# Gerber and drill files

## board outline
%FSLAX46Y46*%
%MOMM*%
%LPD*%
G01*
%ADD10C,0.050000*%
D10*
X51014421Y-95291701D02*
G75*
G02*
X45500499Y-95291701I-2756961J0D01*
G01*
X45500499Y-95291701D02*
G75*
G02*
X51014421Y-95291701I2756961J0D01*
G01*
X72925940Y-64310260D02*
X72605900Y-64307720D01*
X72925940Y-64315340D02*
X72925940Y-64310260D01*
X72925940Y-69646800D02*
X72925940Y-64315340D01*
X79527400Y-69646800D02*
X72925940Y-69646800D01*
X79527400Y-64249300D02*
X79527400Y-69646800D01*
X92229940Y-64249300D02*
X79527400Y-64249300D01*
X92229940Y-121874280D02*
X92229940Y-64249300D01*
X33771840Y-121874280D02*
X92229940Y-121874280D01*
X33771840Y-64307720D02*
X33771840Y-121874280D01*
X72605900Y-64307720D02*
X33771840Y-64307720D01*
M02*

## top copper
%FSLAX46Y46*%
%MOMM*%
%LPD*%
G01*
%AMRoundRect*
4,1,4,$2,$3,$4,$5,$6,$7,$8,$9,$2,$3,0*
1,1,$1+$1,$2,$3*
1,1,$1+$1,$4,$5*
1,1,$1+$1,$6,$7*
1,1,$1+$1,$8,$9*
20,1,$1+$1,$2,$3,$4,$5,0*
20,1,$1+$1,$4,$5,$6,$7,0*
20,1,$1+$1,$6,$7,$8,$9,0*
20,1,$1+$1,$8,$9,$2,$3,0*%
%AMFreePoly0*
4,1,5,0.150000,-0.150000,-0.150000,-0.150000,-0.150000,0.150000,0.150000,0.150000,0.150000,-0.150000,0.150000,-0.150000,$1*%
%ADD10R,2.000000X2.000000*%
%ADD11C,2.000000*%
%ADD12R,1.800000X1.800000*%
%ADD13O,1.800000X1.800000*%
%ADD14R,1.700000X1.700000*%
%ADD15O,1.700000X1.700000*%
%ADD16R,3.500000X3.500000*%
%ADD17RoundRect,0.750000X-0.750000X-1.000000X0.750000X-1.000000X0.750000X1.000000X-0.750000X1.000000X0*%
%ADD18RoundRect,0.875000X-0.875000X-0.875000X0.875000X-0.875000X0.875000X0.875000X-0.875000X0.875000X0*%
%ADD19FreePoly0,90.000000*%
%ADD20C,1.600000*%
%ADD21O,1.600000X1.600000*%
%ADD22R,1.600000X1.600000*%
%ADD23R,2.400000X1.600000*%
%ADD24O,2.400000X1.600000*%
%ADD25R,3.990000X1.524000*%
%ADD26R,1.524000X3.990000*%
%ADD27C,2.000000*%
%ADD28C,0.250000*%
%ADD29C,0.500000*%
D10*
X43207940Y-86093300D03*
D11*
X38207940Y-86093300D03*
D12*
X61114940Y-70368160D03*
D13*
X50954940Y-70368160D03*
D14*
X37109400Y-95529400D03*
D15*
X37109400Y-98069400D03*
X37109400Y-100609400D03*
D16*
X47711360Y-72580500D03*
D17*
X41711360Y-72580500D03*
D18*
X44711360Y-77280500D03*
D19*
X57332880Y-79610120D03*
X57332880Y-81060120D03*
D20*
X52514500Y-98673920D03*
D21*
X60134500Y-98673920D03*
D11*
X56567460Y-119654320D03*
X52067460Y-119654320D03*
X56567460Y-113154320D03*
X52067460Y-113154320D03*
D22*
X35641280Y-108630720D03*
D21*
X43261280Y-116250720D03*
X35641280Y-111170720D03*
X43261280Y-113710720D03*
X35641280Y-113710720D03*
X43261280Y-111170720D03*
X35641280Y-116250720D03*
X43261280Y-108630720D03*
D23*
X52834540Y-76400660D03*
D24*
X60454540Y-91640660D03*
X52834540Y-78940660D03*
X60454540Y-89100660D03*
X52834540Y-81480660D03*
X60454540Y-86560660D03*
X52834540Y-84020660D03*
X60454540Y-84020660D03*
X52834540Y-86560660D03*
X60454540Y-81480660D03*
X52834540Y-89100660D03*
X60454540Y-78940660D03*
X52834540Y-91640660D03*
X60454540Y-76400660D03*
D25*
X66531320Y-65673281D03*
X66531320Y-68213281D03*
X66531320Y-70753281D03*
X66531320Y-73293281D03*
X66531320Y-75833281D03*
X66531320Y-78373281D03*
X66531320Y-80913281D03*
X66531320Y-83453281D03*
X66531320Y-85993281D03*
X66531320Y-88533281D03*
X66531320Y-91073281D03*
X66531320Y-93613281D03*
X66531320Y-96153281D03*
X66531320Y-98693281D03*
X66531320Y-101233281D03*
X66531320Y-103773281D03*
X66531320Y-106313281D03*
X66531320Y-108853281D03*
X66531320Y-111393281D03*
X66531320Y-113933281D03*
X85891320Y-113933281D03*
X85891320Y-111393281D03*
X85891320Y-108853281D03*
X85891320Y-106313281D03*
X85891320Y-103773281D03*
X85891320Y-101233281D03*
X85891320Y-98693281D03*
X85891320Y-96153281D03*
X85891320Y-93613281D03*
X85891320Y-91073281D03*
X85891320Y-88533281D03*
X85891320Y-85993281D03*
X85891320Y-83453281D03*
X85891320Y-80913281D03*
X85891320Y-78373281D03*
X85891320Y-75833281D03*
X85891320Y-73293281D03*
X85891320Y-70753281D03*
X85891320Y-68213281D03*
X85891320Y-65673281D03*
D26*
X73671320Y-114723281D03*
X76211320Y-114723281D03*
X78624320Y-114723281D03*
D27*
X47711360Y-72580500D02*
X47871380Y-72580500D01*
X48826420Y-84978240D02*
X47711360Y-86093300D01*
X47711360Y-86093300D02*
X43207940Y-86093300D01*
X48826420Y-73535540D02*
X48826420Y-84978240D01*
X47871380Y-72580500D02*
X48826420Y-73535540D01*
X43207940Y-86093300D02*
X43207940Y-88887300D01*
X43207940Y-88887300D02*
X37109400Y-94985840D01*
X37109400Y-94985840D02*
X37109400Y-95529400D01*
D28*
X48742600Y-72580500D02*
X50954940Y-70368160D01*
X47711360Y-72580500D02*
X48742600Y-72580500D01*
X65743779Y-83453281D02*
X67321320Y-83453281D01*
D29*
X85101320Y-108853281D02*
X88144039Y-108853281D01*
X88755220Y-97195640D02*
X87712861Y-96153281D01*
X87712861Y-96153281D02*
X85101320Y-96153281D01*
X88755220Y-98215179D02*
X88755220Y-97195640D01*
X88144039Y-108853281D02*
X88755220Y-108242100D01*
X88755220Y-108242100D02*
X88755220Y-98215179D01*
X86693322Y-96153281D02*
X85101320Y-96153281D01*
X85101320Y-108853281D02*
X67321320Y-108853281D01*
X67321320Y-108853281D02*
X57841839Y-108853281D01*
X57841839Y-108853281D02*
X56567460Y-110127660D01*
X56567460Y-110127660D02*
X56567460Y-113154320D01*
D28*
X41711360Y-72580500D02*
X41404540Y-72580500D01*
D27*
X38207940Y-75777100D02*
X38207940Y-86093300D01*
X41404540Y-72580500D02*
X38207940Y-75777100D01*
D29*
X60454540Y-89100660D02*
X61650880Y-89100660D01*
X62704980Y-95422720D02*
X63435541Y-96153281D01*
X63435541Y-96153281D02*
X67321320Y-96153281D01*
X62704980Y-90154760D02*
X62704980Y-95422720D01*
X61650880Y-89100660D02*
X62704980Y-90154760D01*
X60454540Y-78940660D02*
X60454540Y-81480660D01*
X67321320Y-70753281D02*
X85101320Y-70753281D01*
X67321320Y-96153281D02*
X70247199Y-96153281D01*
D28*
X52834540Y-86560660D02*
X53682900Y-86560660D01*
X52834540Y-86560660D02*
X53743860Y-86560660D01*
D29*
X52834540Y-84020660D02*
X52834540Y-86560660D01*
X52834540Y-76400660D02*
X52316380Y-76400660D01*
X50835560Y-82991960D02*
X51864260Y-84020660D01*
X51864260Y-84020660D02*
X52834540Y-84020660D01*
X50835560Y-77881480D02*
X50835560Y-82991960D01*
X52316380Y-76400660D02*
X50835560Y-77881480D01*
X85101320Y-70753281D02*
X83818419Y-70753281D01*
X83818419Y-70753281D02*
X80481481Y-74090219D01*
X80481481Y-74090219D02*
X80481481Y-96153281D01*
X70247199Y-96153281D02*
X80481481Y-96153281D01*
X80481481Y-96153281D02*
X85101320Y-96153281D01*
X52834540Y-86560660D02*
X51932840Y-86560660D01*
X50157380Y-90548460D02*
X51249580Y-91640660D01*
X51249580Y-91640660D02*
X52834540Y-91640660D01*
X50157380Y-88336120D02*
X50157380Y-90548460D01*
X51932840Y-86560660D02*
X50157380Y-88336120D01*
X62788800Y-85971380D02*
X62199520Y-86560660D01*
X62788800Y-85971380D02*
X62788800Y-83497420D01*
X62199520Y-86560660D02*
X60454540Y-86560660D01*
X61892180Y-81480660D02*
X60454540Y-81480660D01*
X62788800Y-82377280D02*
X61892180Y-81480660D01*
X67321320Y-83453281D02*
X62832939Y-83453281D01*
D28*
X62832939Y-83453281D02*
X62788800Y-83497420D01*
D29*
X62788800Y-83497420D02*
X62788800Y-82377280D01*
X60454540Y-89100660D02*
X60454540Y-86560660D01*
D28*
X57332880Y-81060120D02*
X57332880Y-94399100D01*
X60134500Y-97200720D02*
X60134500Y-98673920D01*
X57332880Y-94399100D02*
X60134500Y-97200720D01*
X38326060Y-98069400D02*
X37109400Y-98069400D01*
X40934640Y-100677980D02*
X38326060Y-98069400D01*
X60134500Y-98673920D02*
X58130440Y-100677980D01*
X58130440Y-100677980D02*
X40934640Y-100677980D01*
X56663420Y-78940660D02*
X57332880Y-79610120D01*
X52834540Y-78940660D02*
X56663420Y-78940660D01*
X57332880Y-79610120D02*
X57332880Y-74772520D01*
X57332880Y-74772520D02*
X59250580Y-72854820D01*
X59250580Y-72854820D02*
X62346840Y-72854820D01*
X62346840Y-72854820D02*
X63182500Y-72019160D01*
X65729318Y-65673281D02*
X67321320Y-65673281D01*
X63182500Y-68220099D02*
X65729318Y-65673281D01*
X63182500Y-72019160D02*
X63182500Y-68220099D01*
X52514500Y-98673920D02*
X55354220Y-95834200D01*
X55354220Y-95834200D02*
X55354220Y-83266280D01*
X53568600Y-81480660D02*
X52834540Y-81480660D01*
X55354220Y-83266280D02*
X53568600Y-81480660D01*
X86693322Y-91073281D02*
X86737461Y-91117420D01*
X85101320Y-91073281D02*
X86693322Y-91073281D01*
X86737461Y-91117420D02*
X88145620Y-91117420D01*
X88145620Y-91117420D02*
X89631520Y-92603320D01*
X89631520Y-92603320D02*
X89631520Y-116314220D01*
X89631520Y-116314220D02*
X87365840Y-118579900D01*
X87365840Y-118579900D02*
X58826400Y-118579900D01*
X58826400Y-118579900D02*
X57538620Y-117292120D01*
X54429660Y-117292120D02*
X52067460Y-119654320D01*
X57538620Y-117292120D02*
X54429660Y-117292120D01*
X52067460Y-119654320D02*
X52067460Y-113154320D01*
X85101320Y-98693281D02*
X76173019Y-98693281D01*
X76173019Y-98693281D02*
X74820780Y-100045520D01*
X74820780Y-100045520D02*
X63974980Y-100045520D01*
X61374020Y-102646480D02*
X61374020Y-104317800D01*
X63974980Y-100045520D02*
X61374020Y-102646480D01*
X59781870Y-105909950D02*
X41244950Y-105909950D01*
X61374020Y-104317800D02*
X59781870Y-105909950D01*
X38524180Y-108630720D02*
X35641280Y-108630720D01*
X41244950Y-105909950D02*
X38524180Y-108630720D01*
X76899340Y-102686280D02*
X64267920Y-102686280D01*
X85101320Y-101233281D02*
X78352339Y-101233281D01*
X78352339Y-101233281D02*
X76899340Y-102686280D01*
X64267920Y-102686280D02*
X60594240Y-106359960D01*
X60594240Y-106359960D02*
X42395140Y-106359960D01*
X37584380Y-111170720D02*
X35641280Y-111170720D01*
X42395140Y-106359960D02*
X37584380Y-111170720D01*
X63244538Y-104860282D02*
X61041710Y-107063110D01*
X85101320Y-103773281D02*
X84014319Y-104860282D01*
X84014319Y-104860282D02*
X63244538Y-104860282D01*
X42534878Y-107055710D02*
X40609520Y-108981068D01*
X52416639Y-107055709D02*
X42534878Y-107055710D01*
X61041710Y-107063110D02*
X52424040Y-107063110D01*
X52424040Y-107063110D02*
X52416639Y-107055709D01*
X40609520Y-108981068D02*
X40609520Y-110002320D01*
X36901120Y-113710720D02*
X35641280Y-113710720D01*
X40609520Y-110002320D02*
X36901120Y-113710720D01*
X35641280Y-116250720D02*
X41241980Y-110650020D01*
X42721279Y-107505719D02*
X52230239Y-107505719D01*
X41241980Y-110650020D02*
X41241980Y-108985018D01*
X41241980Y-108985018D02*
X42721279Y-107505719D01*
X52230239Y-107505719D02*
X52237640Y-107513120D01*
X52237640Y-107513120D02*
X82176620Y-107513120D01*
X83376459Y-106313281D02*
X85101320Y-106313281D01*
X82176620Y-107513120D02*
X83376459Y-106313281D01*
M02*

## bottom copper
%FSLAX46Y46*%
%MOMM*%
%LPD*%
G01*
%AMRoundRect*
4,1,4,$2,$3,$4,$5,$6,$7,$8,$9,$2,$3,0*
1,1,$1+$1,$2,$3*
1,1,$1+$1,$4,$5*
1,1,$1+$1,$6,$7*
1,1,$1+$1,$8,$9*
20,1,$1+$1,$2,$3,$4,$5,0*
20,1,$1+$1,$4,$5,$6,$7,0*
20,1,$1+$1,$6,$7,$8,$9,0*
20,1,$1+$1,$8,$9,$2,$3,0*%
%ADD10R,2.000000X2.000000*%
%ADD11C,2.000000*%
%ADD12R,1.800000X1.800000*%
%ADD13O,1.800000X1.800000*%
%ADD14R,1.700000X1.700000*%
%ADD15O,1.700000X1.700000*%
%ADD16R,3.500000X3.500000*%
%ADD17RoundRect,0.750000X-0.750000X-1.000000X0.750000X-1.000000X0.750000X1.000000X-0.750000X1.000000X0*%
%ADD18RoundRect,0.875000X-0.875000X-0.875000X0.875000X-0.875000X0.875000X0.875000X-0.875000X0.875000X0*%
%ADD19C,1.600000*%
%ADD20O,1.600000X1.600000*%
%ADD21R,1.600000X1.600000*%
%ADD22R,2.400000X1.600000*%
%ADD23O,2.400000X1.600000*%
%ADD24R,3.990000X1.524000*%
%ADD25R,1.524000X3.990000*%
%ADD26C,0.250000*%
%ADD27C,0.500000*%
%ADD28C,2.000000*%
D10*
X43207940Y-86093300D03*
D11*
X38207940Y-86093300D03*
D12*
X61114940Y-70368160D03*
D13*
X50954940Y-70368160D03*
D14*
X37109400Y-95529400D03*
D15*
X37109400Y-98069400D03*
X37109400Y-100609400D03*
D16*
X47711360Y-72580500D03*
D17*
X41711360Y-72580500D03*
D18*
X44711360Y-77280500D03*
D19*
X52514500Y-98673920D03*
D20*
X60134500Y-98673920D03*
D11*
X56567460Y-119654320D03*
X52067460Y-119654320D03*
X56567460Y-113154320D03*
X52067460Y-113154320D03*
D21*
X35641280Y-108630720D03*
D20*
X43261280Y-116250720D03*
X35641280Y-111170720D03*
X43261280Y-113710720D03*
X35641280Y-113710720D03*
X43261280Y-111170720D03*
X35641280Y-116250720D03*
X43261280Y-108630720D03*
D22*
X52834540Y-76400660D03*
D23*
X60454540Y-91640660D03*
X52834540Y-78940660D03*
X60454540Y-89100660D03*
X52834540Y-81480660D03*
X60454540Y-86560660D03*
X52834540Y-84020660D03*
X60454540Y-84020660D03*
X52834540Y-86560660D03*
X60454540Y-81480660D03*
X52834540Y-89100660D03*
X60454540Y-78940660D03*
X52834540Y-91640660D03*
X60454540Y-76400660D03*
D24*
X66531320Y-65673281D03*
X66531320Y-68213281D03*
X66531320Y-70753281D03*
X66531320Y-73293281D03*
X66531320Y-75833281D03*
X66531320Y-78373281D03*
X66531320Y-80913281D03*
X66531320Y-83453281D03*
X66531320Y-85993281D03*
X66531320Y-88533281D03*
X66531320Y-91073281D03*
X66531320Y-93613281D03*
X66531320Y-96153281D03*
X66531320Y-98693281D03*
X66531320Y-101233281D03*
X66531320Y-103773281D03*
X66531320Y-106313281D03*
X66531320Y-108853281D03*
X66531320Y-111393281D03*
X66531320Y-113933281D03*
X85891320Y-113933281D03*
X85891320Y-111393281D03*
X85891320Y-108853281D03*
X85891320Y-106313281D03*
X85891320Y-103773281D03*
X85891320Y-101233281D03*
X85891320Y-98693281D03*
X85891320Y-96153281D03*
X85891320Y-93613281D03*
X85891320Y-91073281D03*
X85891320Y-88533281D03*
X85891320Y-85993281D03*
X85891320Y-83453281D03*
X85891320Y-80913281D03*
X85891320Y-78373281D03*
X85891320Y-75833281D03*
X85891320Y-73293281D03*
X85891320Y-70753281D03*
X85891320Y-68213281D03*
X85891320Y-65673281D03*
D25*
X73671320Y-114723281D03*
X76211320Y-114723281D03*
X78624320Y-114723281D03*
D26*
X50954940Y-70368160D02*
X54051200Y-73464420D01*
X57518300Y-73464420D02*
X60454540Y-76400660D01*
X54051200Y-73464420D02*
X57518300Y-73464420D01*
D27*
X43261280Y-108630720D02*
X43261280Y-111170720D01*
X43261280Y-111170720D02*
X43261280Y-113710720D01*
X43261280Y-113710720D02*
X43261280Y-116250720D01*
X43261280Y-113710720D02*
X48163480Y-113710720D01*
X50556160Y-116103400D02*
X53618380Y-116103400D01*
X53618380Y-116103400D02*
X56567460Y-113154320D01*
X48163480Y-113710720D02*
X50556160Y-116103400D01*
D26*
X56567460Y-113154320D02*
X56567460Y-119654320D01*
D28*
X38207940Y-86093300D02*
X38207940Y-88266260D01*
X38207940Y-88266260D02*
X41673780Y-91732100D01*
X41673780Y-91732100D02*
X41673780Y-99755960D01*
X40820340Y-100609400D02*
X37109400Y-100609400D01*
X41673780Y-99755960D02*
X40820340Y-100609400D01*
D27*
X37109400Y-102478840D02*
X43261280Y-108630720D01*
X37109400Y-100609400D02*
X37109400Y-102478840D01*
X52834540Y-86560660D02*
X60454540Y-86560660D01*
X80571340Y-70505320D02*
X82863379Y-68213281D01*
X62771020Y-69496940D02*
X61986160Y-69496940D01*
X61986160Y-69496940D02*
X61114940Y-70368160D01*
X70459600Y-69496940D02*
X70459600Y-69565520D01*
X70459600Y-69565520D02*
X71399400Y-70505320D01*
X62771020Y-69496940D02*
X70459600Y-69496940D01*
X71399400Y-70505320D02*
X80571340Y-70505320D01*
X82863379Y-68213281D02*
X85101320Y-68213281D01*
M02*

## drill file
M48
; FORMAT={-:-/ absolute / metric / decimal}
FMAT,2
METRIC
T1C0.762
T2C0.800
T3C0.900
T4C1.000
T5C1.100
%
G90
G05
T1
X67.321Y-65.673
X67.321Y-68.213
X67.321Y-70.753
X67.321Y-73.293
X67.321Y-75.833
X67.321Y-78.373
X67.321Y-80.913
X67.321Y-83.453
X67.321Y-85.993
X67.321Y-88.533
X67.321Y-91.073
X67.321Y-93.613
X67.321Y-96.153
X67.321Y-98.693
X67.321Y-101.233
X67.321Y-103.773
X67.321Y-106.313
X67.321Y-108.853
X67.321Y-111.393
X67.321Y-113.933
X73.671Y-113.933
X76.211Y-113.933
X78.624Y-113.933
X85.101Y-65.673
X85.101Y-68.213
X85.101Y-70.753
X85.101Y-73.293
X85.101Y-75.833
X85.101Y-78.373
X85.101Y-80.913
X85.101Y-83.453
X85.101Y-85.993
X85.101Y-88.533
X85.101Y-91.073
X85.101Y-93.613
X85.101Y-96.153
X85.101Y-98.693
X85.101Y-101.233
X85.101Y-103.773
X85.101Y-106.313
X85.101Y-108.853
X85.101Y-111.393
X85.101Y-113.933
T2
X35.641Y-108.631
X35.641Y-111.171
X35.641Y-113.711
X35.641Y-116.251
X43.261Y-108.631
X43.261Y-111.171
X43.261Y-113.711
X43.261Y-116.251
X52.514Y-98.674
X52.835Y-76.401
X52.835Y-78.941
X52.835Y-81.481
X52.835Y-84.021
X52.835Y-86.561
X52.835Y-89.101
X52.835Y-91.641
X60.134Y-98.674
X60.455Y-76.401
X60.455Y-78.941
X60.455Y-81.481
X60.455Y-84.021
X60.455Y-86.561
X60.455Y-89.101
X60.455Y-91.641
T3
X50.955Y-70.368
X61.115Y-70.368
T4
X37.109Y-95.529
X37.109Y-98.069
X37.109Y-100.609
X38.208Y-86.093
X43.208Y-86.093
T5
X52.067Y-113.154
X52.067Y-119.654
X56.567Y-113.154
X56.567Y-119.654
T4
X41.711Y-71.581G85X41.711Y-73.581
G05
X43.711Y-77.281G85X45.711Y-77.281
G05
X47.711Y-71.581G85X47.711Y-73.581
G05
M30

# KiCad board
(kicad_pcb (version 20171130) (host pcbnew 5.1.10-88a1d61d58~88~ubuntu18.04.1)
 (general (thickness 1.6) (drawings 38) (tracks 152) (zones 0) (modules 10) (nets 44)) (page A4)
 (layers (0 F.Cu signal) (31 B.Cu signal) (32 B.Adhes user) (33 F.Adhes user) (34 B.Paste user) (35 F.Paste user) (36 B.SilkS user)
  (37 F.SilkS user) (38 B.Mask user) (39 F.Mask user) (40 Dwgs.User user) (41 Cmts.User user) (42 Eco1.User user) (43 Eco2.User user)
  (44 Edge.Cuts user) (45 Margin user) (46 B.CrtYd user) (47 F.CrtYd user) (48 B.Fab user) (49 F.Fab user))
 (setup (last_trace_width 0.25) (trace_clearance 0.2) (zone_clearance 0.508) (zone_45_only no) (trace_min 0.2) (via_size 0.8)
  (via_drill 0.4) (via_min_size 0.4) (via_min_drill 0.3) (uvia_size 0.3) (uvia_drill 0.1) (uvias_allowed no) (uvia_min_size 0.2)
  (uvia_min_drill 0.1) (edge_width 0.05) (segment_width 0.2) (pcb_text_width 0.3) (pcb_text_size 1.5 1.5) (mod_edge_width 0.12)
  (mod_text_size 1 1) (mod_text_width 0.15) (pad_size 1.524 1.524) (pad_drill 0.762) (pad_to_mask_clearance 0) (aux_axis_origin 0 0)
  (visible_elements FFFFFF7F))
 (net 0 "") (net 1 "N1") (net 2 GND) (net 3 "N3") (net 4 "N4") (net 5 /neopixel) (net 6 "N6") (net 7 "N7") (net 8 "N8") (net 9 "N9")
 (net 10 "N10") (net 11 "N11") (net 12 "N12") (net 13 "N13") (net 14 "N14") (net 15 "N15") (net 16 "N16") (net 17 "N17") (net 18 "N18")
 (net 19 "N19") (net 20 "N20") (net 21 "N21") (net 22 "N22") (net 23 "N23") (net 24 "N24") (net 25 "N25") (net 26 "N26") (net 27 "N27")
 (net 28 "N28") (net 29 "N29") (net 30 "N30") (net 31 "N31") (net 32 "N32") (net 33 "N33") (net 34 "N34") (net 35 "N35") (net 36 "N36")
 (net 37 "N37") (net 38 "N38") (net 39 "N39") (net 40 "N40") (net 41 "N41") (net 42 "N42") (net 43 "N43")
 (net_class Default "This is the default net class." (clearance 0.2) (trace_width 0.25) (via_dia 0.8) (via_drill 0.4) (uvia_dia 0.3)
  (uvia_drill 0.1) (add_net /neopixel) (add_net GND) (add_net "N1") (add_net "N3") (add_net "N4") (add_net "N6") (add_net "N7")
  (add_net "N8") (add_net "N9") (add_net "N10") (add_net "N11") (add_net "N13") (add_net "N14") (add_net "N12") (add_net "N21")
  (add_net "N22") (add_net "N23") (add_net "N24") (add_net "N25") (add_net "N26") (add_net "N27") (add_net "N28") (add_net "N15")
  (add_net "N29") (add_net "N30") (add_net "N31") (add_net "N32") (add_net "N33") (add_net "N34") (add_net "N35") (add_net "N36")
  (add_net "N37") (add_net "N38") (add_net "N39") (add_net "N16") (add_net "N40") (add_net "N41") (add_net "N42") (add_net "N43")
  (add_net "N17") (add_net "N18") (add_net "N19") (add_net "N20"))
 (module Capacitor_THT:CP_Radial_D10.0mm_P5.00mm (layer F.Cu) (at 43.20794 86.0933 180)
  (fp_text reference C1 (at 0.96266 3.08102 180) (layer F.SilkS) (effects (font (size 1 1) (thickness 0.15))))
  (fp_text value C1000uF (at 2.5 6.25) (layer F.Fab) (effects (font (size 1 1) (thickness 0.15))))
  (pad 1 thru_hole rect (at 0 0 180) (size 2 2) (drill 1) (layers *.Cu *.Mask) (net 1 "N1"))
  (pad 2 thru_hole circle (at 5 0 180) (size 2 2) (drill 1) (layers *.Cu *.Mask) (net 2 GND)))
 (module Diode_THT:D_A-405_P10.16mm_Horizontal (layer F.Cu) (at 61.11494 70.36816 180)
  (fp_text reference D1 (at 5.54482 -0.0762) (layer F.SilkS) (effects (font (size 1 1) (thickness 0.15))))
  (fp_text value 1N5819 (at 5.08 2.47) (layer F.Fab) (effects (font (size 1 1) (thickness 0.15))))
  (pad 1 thru_hole rect (at 0 0 180) (size 1.8 1.8) (drill 0.9) (layers *.Cu *.Mask) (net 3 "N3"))
  (pad 2 thru_hole oval (at 10.16 0 180) (size 1.8 1.8) (drill 0.9) (layers *.Cu *.Mask) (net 1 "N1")))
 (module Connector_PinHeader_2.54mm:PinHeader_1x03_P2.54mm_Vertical (layer F.Cu) (at 37.1094 95.5294)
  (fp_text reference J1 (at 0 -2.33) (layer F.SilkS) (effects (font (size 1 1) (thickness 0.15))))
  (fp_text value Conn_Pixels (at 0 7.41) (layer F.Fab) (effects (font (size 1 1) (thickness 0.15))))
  (pad 1 thru_hole rect (at 0 0) (size 1.7 1.7) (drill 1) (layers *.Cu *.Mask) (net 1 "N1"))
  (pad 2 thru_hole oval (at 0 2.54) (size 1.7 1.7) (drill 1) (layers *.Cu *.Mask) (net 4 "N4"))
  (pad 3 thru_hole oval (at 0 5.08) (size 1.7 1.7) (drill 1) (layers *.Cu *.Mask) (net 2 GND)))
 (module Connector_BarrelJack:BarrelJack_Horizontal (layer F.Cu) (at 47.71136 72.5805)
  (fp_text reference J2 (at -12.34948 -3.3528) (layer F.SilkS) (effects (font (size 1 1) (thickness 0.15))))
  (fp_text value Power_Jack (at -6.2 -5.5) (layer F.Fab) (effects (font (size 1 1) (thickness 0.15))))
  (pad 1 thru_hole rect (at 0 0) (size 3.5 3.5) (drill oval 1 3) (layers *.Cu *.Mask) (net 1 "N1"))
  (pad 2 thru_hole roundrect (at -6 0) (size 3 3.5) (drill oval 1 3) (layers *.Cu *.Mask) (roundrect_rratio 0.25) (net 2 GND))
  (pad 3 thru_hole roundrect (at -3 4.7) (size 3.5 3.5) (drill oval 3 1) (layers *.Cu *.Mask) (roundrect_rratio 0.25)))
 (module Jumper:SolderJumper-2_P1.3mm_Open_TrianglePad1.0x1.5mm (layer F.Cu) (at 57.33288 80.33512 90)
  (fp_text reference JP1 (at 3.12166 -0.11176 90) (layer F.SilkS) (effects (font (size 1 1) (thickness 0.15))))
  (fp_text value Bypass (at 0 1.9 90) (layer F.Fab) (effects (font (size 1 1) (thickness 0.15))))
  (pad 2 smd custom (at 0.725 0 90) (size 0.3 0.3) (layers F.Cu F.Mask) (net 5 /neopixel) (zone_connect 2)
   (options (clearance outline) (anchor rect)) (primitives))
  (pad 1 smd custom (at -0.725 0 90) (size 0.3 0.3) (layers F.Cu F.Mask) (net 4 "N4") (zone_connect 2)
   (options (clearance outline) (anchor rect)) (primitives)))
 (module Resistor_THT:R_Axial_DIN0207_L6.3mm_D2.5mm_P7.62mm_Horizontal (layer F.Cu) (at 52.5145 98.67392)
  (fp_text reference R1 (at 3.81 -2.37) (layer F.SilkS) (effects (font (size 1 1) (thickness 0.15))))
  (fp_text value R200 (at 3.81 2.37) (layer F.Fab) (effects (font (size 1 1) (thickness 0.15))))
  (pad 1 thru_hole circle (at 0 0) (size 1.6 1.6) (drill 0.8) (layers *.Cu *.Mask) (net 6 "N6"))
  (pad 2 thru_hole oval (at 7.62 0) (size 1.6 1.6) (drill 0.8) (layers *.Cu *.Mask) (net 4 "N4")))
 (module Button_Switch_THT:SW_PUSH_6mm (layer F.Cu) (at 52.06746 119.65432 90)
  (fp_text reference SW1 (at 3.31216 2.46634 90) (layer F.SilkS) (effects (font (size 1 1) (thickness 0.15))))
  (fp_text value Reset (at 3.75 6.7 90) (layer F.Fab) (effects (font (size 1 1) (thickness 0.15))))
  (pad 2 thru_hole circle (at 0 4.5 180) (size 2 2) (drill 1.1) (layers *.Cu *.Mask) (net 2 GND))
  (pad 1 thru_hole circle (at 0 0 180) (size 2 2) (drill 1.1) (layers *.Cu *.Mask) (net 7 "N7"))
  (pad 2 thru_hole circle (at 6.5 4.5 180) (size 2 2) (drill 1.1) (layers *.Cu *.Mask) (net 2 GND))
  (pad 1 thru_hole circle (at 6.5 0 180) (size 2 2) (drill 1.1) (layers *.Cu *.Mask) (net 7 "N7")))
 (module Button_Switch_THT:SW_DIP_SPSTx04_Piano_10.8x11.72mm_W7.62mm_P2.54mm (layer F.Cu) (at 35.64128 108.63072)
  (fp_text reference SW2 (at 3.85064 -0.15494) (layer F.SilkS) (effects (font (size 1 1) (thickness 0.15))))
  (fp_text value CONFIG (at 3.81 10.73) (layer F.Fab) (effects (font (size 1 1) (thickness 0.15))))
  (pad 1 thru_hole rect (at 0 0) (size 1.6 1.6) (drill 0.8) (layers *.Cu *.Mask) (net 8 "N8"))
  (pad 5 thru_hole oval (at 7.62 7.62) (size 1.6 1.6) (drill 0.8) (layers *.Cu *.Mask) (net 2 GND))
  (pad 2 thru_hole oval (at 0 2.54) (size 1.6 1.6) (drill 0.8) (layers *.Cu *.Mask) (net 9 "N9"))
  (pad 6 thru_hole oval (at 7.62 5.08) (size 1.6 1.6) (drill 0.8) (layers *.Cu *.Mask) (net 2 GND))
  (pad 3 thru_hole oval (at 0 5.08) (size 1.6 1.6) (drill 0.8) (layers *.Cu *.Mask) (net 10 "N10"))
  (pad 7 thru_hole oval (at 7.62 2.54) (size 1.6 1.6) (drill 0.8) (layers *.Cu *.Mask) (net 2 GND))
  (pad 4 thru_hole oval (at 0 7.62) (size 1.6 1.6) (drill 0.8) (layers *.Cu *.Mask) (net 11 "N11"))
  (pad 8 thru_hole oval (at 7.62 0) (size 1.6 1.6) (drill 0.8) (layers *.Cu *.Mask) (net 2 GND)))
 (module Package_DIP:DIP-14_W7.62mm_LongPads (layer F.Cu) (at 52.83454 76.40066)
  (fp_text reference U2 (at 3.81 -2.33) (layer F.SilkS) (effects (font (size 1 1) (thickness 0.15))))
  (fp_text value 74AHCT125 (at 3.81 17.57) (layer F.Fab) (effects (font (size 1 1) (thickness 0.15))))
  (pad 1 thru_hole rect (at 0 0) (size 2.4 1.6) (drill 0.8) (layers *.Cu *.Mask) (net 2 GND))
  (pad 8 thru_hole oval (at 7.62 15.24) (size 2.4 1.6) (drill 0.8) (layers *.Cu *.Mask) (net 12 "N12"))
  (pad 2 thru_hole oval (at 0 2.54) (size 2.4 1.6) (drill 0.8) (layers *.Cu *.Mask) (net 5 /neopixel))
  (pad 9 thru_hole oval (at 7.62 12.7) (size 2.4 1.6) (drill 0.8) (layers *.Cu *.Mask) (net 2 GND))
  (pad 3 thru_hole oval (at 0 5.08) (size 2.4 1.6) (drill 0.8) (layers *.Cu *.Mask) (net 6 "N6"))
  (pad 10 thru_hole oval (at 7.62 10.16) (size 2.4 1.6) (drill 0.8) (layers *.Cu *.Mask) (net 2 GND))
  (pad 4 thru_hole oval (at 0 7.62) (size 2.4 1.6) (drill 0.8) (layers *.Cu *.Mask) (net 2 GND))
  (pad 11 thru_hole oval (at 7.62 7.62) (size 2.4 1.6) (drill 0.8) (layers *.Cu *.Mask) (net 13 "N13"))
  (pad 5 thru_hole oval (at 0 10.16) (size 2.4 1.6) (drill 0.8) (layers *.Cu *.Mask) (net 2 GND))
  (pad 12 thru_hole oval (at 7.62 5.08) (size 2.4 1.6) (drill 0.8) (layers *.Cu *.Mask) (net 2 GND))
  (pad 6 thru_hole oval (at 0 12.7) (size 2.4 1.6) (drill 0.8) (layers *.Cu *.Mask) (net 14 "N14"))
  (pad 13 thru_hole oval (at 7.62 2.54) (size 2.4 1.6) (drill 0.8) (layers *.Cu *.Mask) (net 2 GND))
  (pad 7 thru_hole oval (at 0 15.24) (size 2.4 1.6) (drill 0.8) (layers *.Cu *.Mask) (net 2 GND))
  (pad 14 thru_hole oval (at 7.62 0) (size 2.4 1.6) (drill 0.8) (layers *.Cu *.Mask) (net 1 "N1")))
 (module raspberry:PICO (layer F.Cu) (at 67.32132 65.673281)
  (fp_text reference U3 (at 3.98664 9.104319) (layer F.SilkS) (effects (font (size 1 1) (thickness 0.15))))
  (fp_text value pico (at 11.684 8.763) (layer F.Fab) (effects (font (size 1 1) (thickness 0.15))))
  (pad 1 thru_hole rect (at 0 0) (size 3.99 1.524) (drill 0.762 (offset -0.79 0)) (layers *.Cu *.Mask) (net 5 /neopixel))
  (pad 2 thru_hole rect (at 0 2.54) (size 3.99 1.524) (drill 0.762 (offset -0.79 0)) (layers *.Cu *.Mask) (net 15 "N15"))
  (pad 3 thru_hole rect (at 0 5.08) (size 3.99 1.524) (drill 0.762 (offset -0.79 0)) (layers *.Cu *.Mask) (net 2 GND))
  (pad 4 thru_hole rect (at 0 7.62) (size 3.99 1.524) (drill 0.762 (offset -0.79 0)) (layers *.Cu *.Mask) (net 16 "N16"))
  (pad 5 thru_hole rect (at 0 10.16) (size 3.99 1.524) (drill 0.762 (offset -0.79 0)) (layers *.Cu *.Mask) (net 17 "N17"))
  (pad 6 thru_hole rect (at 0 12.7) (size 3.99 1.524) (drill 0.762 (offset -0.79 0)) (layers *.Cu *.Mask) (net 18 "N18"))
  (pad 7 thru_hole rect (at 0 15.24) (size 3.99 1.524) (drill 0.762 (offset -0.79 0)) (layers *.Cu *.Mask) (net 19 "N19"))
  (pad 8 thru_hole rect (at 0 17.78) (size 3.99 1.524) (drill 0.762 (offset -0.79 0)) (layers *.Cu *.Mask) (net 2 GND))
  (pad 9 thru_hole rect (at 0 20.32) (size 3.99 1.524) (drill 0.762 (offset -0.79 0)) (layers *.Cu *.Mask) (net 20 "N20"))
  (pad 10 thru_hole rect (at 0 22.86) (size 3.99 1.524) (drill 0.762 (offset -0.79 0)) (layers *.Cu *.Mask) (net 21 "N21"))
  (pad 11 thru_hole rect (at 0 25.4) (size 3.99 1.524) (drill 0.762 (offset -0.79 0)) (layers *.Cu *.Mask) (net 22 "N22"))
  (pad 12 thru_hole rect (at 0 27.94) (size 3.99 1.524) (drill 0.762 (offset -0.79 0)) (layers *.Cu *.Mask) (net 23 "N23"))
  (pad 13 thru_hole rect (at 0 30.48) (size 3.99 1.524) (drill 0.762 (offset -0.79 0)) (layers *.Cu *.Mask) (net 2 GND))
  (pad 14 thru_hole rect (at 0 33.02) (size 3.99 1.524) (drill 0.762 (offset -0.79 0)) (layers *.Cu *.Mask) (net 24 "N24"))
  (pad 15 thru_hole rect (at 0 35.56) (size 3.99 1.524) (drill 0.762 (offset -0.79 0)) (layers *.Cu *.Mask) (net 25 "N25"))
  (pad 16 thru_hole rect (at 0 38.1) (size 3.99 1.524) (drill 0.762 (offset -0.79 0)) (layers *.Cu *.Mask) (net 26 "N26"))
  (pad 17 thru_hole rect (at 0 40.64) (size 3.99 1.524) (drill 0.762 (offset -0.79 0)) (layers *.Cu *.Mask) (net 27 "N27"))
  (pad 18 thru_hole rect (at 0 43.18) (size 3.99 1.524) (drill 0.762 (offset -0.79 0)) (layers *.Cu *.Mask) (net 2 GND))
  (pad 19 thru_hole rect (at 0 45.72) (size 3.99 1.524) (drill 0.762 (offset -0.79 0)) (layers *.Cu *.Mask) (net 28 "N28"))
  (pad 20 thru_hole rect (at 0 48.26) (size 3.99 1.524) (drill 0.762 (offset -0.79 0)) (layers *.Cu *.Mask) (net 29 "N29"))
  (pad 21 thru_hole rect (at 17.78 48.26) (size 3.99 1.524) (drill 0.762 (offset 0.79 0)) (layers *.Cu *.Mask) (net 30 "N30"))
  (pad 22 thru_hole rect (at 17.78 45.72) (size 3.99 1.524) (drill 0.762 (offset 0.79 0)) (layers *.Cu *.Mask) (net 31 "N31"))
  (pad 23 thru_hole rect (at 17.78 43.18) (size 3.99 1.524) (drill 0.762 (offset 0.79 0)) (layers *.Cu *.Mask) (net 2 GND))
  (pad 24 thru_hole rect (at 17.78 40.64) (size 3.99 1.524) (drill 0.762 (offset 0.79 0)) (layers *.Cu *.Mask) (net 11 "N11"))
  (pad 25 thru_hole rect (at 17.78 38.1) (size 3.99 1.524) (drill 0.762 (offset 0.79 0)) (layers *.Cu *.Mask) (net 10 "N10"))
  (pad 26 thru_hole rect (at 17.78 35.56) (size 3.99 1.524) (drill 0.762 (offset 0.79 0)) (layers *.Cu *.Mask) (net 9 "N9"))
  (pad 27 thru_hole rect (at 17.78 33.02) (size 3.99 1.524) (drill 0.762 (offset 0.79 0)) (layers *.Cu *.Mask) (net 8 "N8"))
  (pad 28 thru_hole rect (at 17.78 30.48) (size 3.99 1.524) (drill 0.762 (offset 0.79 0)) (layers *.Cu *.Mask) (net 2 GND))
  (pad 29 thru_hole rect (at 17.78 27.94) (size 3.99 1.524) (drill 0.762 (offset 0.79 0)) (layers *.Cu *.Mask) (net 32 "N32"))
  (pad 30 thru_hole rect (at 17.78 25.4) (size 3.99 1.524) (drill 0.762 (offset 0.79 0)) (layers *.Cu *.Mask) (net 7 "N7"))
  (pad 31 thru_hole rect (at 17.78 22.86) (size 3.99 1.524) (drill 0.762 (offset 0.79 0)) (layers *.Cu *.Mask) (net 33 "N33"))
  (pad 32 thru_hole rect (at 17.78 20.32) (size 3.99 1.524) (drill 0.762 (offset 0.79 0)) (layers *.Cu *.Mask) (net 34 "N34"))
  (pad 33 thru_hole rect (at 17.78 17.78) (size 3.99 1.524) (drill 0.762 (offset 0.79 0)) (layers *.Cu *.Mask) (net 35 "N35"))
  (pad 34 thru_hole rect (at 17.78 15.24) (size 3.99 1.524) (drill 0.762 (offset 0.79 0)) (layers *.Cu *.Mask) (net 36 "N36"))
  (pad 35 thru_hole rect (at 17.78 12.7) (size 3.99 1.524) (drill 0.762 (offset 0.79 0)) (layers *.Cu *.Mask) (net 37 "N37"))
  (pad 36 thru_hole rect (at 17.78 10.16) (size 3.99 1.524) (drill 0.762 (offset 0.79 0)) (layers *.Cu *.Mask) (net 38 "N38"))
  (pad 37 thru_hole rect (at 17.78 7.62) (size 3.99 1.524) (drill 0.762 (offset 0.79 0)) (layers *.Cu *.Mask) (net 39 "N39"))
  (pad 38 thru_hole rect (at 17.78 5.08) (size 3.99 1.524) (drill 0.762 (offset 0.79 0)) (layers *.Cu *.Mask) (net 2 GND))
  (pad 39 thru_hole rect (at 17.78 2.54) (size 3.99 1.524) (drill 0.762 (offset 0.79 0)) (layers *.Cu *.Mask) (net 3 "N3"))
  (pad 40 thru_hole rect (at 17.78 0) (size 3.99 1.524) (drill 0.762 (offset 0.79 0)) (layers *.Cu *.Mask) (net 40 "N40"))
  (pad 41 thru_hole rect (at 6.35 48.26 270) (size 3.99 1.524) (drill 0.762 (offset 0.79 0)) (layers *.Cu *.Mask) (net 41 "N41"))
  (pad 42 thru_hole rect (at 8.89 48.26 270) (size 3.99 1.524) (drill 0.762 (offset 0.79 0)) (layers *.Cu *.Mask) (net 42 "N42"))
  (pad 43 thru_hole rect (at 11.303 48.26 270) (size 3.99 1.524) (drill 0.762 (offset 0.79 0)) (layers *.Cu *.Mask) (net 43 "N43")))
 (gr_circle (center 48.25746 95.291701) (end 50.78222 96.399141) (layer Edge.Cuts) (width 0.05))
 (gr_line (start 72.92594 64.31026) (end 72.6059 64.30772) (layer Edge.Cuts) (width 0.05))
 (gr_line (start 72.92594 64.31534) (end 72.92594 64.31026) (layer Edge.Cuts) (width 0.05))
 (gr_line (start 72.92594 69.6468) (end 72.92594 64.31534) (layer Edge.Cuts) (width 0.05))
 (gr_line (start 79.5274 69.6468) (end 72.92594 69.6468) (layer Edge.Cuts) (width 0.05))
 (gr_line (start 79.5274 64.2493) (end 79.5274 69.6468) (layer Edge.Cuts) (width 0.05))
 (gr_line (start 92.22994 64.2493) (end 79.5274 64.2493) (layer Edge.Cuts) (width 0.05))
 (gr_line (start 92.22994 121.87428) (end 92.22994 64.2493) (layer Edge.Cuts) (width 0.05))
 (gr_line (start 33.77184 121.87428) (end 92.22994 121.87428) (layer Edge.Cuts) (width 0.05))
 (gr_line (start 33.77184 64.30772) (end 33.77184 121.87428) (layer Edge.Cuts) (width 0.05))
 (gr_line (start 72.6059 64.30772) (end 33.77184 64.30772) (layer Edge.Cuts) (width 0.05))
 (segment (start 47.71136 72.5805) (end 47.87138 72.5805) (width 2) (layer F.Cu) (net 1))
 (segment (start 48.82642 84.97824) (end 47.71136 86.0933) (width 2) (layer F.Cu) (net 1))
 (segment (start 47.71136 86.0933) (end 43.20794 86.0933) (width 2) (layer F.Cu) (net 1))
 (segment (start 48.82642 73.53554) (end 48.82642 84.97824) (width 2) (layer F.Cu) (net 1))
 (segment (start 47.87138 72.5805) (end 48.82642 73.53554) (width 2) (layer F.Cu) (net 1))
 (segment (start 43.20794 86.0933) (end 43.20794 88.8873) (width 2) (layer F.Cu) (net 1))
 (segment (start 43.20794 88.8873) (end 37.1094 94.98584) (width 2) (layer F.Cu) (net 1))
 (segment (start 37.1094 94.98584) (end 37.1094 95.5294) (width 2) (layer F.Cu) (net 1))
 (segment (start 48.7426 72.5805) (end 50.95494 70.36816) (width 0.25) (layer F.Cu) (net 1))
 (segment (start 47.71136 72.5805) (end 48.7426 72.5805) (width 0.25) (layer F.Cu) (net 1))
 (segment (start 50.95494 70.36816) (end 54.0512 73.46442) (width 0.25) (layer B.Cu) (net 1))
 (segment (start 57.5183 73.46442) (end 60.45454 76.40066) (width 0.25) (layer B.Cu) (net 1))
 (segment (start 54.0512 73.46442) (end 57.5183 73.46442) (width 0.25) (layer B.Cu) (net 1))
 (segment (start 43.26128 108.63072) (end 43.26128 111.17072) (width 0.5) (layer B.Cu) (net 2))
 (segment (start 43.26128 111.17072) (end 43.26128 113.71072) (width 0.5) (layer B.Cu) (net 2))
 (segment (start 43.26128 113.71072) (end 43.26128 116.25072) (width 0.5) (layer B.Cu) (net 2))
 (segment (start 43.26128 113.71072) (end 48.16348 113.71072) (width 0.5) (layer B.Cu) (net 2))
 (segment (start 50.55616 116.1034) (end 53.61838 116.1034) (width 0.5) (layer B.Cu) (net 2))
 (segment (start 53.61838 116.1034) (end 56.56746 113.15432) (width 0.5) (layer B.Cu) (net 2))
 (segment (start 48.16348 113.71072) (end 50.55616 116.1034) (width 0.5) (layer B.Cu) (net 2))
 (segment (start 56.56746 113.15432) (end 56.56746 119.65432) (width 0.25) (layer B.Cu) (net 2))
 (segment (start 65.743779 83.453281) (end 67.32132 83.453281) (width 0.25) (layer F.Cu) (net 2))
 (segment (start 85.10132 108.853281) (end 88.144039 108.853281) (width 0.5) (layer F.Cu) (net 2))
 (segment (start 88.75522 97.19564) (end 87.712861 96.153281) (width 0.5) (layer F.Cu) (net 2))
 (segment (start 87.712861 96.153281) (end 85.10132 96.153281) (width 0.5) (layer F.Cu) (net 2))
 (segment (start 88.75522 98.215179) (end 88.75522 97.19564) (width 0.5) (layer F.Cu) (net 2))
 (segment (start 88.144039 108.853281) (end 88.75522 108.2421) (width 0.5) (layer F.Cu) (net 2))
 (segment (start 88.75522 108.2421) (end 88.75522 98.215179) (width 0.5) (layer F.Cu) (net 2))
 (segment (start 86.693322 96.153281) (end 85.10132 96.153281) (width 0.5) (layer F.Cu) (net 2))
 (segment (start 85.10132 108.853281) (end 67.32132 108.853281) (width 0.5) (layer F.Cu) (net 2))
 (segment (start 67.32132 108.853281) (end 57.841839 108.853281) (width 0.5) (layer F.Cu) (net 2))
 (segment (start 57.841839 108.853281) (end 56.56746 110.12766) (width 0.5) (layer F.Cu) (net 2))
 (segment (start 56.56746 110.12766) (end 56.56746 113.15432) (width 0.5) (layer F.Cu) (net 2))
 (segment (start 41.71136 72.5805) (end 41.40454 72.5805) (width 0.25) (layer F.Cu) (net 2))
 (segment (start 38.20794 75.7771) (end 38.20794 86.0933) (width 2) (layer F.Cu) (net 2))
 (segment (start 41.40454 72.5805) (end 38.20794 75.7771) (width 2) (layer F.Cu) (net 2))
 (segment (start 38.20794 86.0933) (end 38.20794 88.26626) (width 2) (layer B.Cu) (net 2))
 (segment (start 38.20794 88.26626) (end 41.67378 91.7321) (width 2) (layer B.Cu) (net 2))
 (segment (start 41.67378 91.7321) (end 41.67378 99.75596) (width 2) (layer B.Cu) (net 2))
 (segment (start 40.82034 100.6094) (end 37.1094 100.6094) (width 2) (layer B.Cu) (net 2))
 (segment (start 41.67378 99.75596) (end 40.82034 100.6094) (width 2) (layer B.Cu) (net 2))
 (segment (start 37.1094 102.47884) (end 43.26128 108.63072) (width 0.5) (layer B.Cu) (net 2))
 (segment (start 37.1094 100.6094) (end 37.1094 102.47884) (width 0.5) (layer B.Cu) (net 2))
 (segment (start 60.45454 89.10066) (end 61.65088 89.10066) (width 0.5) (layer F.Cu) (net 2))
 (segment (start 62.70498 95.42272) (end 63.435541 96.153281) (width 0.5) (layer F.Cu) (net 2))
 (segment (start 63.435541 96.153281) (end 67.32132 96.153281) (width 0.5) (layer F.Cu) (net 2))
 (segment (start 62.70498 90.15476) (end 62.70498 95.42272) (width 0.5) (layer F.Cu) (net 2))
 (segment (start 61.65088 89.10066) (end 62.70498 90.15476) (width 0.5) (layer F.Cu) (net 2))
 (segment (start 60.45454 78.94066) (end 60.45454 81.48066) (width 0.5) (layer F.Cu) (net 2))
 (segment (start 67.32132 70.753281) (end 85.10132 70.753281) (width 0.5) (layer F.Cu) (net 2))
 (segment (start 67.32132 96.153281) (end 70.247199 96.153281) (width 0.5) (layer F.Cu) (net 2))
 (segment (start 52.83454 86.56066) (end 53.6829 86.56066) (width 0.25) (layer F.Cu) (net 2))
 (segment (start 52.83454 86.56066) (end 53.74386 86.56066) (width 0.25) (layer F.Cu) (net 2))
 (segment (start 52.83454 84.02066) (end 52.83454 86.56066) (width 0.5) (layer F.Cu) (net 2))
 (segment (start 52.83454 76.40066) (end 52.31638 76.40066) (width 0.5) (layer F.Cu) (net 2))
 (segment (start 50.83556 82.99196) (end 51.86426 84.02066) (width 0.5) (layer F.Cu) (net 2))
 (segment (start 51.86426 84.02066) (end 52.83454 84.02066) (width 0.5) (layer F.Cu) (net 2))
 (segment (start 50.83556 77.88148) (end 50.83556 82.99196) (width 0.5) (layer F.Cu) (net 2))
 (segment (start 52.31638 76.40066) (end 50.83556 77.88148) (width 0.5) (layer F.Cu) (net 2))
 (segment (start 85.10132 70.753281) (end 83.818419 70.753281) (width 0.5) (layer F.Cu) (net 2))
 (segment (start 83.818419 70.753281) (end 80.481481 74.090219) (width 0.5) (layer F.Cu) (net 2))
 (segment (start 80.481481 74.090219) (end 80.481481 96.153281) (width 0.5) (layer F.Cu) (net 2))
 (segment (start 70.247199 96.153281) (end 80.481481 96.153281) (width 0.5) (layer F.Cu) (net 2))
 (segment (start 80.481481 96.153281) (end 85.10132 96.153281) (width 0.5) (layer F.Cu) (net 2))
 (segment (start 52.83454 86.56066) (end 51.93284 86.56066) (width 0.5) (layer F.Cu) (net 2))
 (segment (start 50.15738 90.54846) (end 51.24958 91.64066) (width 0.5) (layer F.Cu) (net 2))
 (segment (start 51.24958 91.64066) (end 52.83454 91.64066) (width 0.5) (layer F.Cu) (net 2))
 (segment (start 50.15738 88.33612) (end 50.15738 90.54846) (width 0.5) (layer F.Cu) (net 2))
 (segment (start 51.93284 86.56066) (end 50.15738 88.33612) (width 0.5) (layer F.Cu) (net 2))
 (segment (start 62.7888 85.97138) (end 62.19952 86.56066) (width 0.5) (layer F.Cu) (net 2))
 (segment (start 62.7888 85.97138) (end 62.7888 83.49742) (width 0.5) (layer F.Cu) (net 2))
 (segment (start 62.19952 86.56066) (end 60.45454 86.56066) (width 0.5) (layer F.Cu) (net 2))
 (segment (start 61.89218 81.48066) (end 60.45454 81.48066) (width 0.5) (layer F.Cu) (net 2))
 (segment (start 62.7888 82.37728) (end 61.89218 81.48066) (width 0.5) (layer F.Cu) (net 2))
 (segment (start 67.32132 83.453281) (end 62.832939 83.453281) (width 0.5) (layer F.Cu) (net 2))
 (segment (start 62.832939 83.453281) (end 62.7888 83.49742) (width 0.25) (layer F.Cu) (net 2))
 (segment (start 62.7888 83.49742) (end 62.7888 82.37728) (width 0.5) (layer F.Cu) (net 2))
 (segment (start 60.45454 89.10066) (end 60.45454 86.56066) (width 0.5) (layer F.Cu) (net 2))
 (segment (start 52.83454 86.56066) (end 60.45454 86.56066) (width 0.5) (layer B.Cu) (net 2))
 (segment (start 80.57134 70.50532) (end 82.863379 68.213281) (width 0.5) (layer B.Cu) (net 3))
 (segment (start 62.77102 69.49694) (end 61.98616 69.49694) (width 0.5) (layer B.Cu) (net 3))
 (segment (start 61.98616 69.49694) (end 61.11494 70.36816) (width 0.5) (layer B.Cu) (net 3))
 (segment (start 70.4596 69.49694) (end 70.4596 69.56552) (width 0.5) (layer B.Cu) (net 3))
 (segment (start 70.4596 69.56552) (end 71.3994 70.50532) (width 0.5) (layer B.Cu) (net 3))
 (segment (start 62.77102 69.49694) (end 70.4596 69.49694) (width 0.5) (layer B.Cu) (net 3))
 (segment (start 71.3994 70.50532) (end 80.57134 70.50532) (width 0.5) (layer B.Cu) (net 3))
 (segment (start 82.863379 68.213281) (end 85.10132 68.213281) (width 0.5) (layer B.Cu) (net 3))
 (segment (start 57.33288 81.06012) (end 57.33288 94.3991) (width 0.25) (layer F.Cu) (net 4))
 (segment (start 60.1345 97.20072) (end 60.1345 98.67392) (width 0.25) (layer F.Cu) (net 4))
 (segment (start 57.33288 94.3991) (end 60.1345 97.20072) (width 0.25) (layer F.Cu) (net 4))
 (segment (start 38.32606 98.0694) (end 37.1094 98.0694) (width 0.25) (layer F.Cu) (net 4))
 (segment (start 40.93464 100.67798) (end 38.32606 98.0694) (width 0.25) (layer F.Cu) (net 4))
 (segment (start 60.1345 98.67392) (end 58.13044 100.67798) (width 0.25) (layer F.Cu) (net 4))
 (segment (start 58.13044 100.67798) (end 40.93464 100.67798) (width 0.25) (layer F.Cu) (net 4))
 (segment (start 56.66342 78.94066) (end 57.33288 79.61012) (width 0.25) (layer F.Cu) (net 5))
 (segment (start 52.83454 78.94066) (end 56.66342 78.94066) (width 0.25) (layer F.Cu) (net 5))
 (segment (start 57.33288 79.61012) (end 57.33288 74.77252) (width 0.25) (layer F.Cu) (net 5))
 (segment (start 57.33288 74.77252) (end 59.25058 72.85482) (width 0.25) (layer F.Cu) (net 5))
 (segment (start 59.25058 72.85482) (end 62.34684 72.85482) (width 0.25) (layer F.Cu) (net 5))
 (segment (start 62.34684 72.85482) (end 63.1825 72.01916) (width 0.25) (layer F.Cu) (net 5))
 (segment (start 65.729318 65.673281) (end 67.32132 65.673281) (width 0.25) (layer F.Cu) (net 5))
 (segment (start 63.1825 68.220099) (end 65.729318 65.673281) (width 0.25) (layer F.Cu) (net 5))
 (segment (start 63.1825 72.01916) (end 63.1825 68.220099) (width 0.25) (layer F.Cu) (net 5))
 (segment (start 52.5145 98.67392) (end 55.35422 95.8342) (width 0.25) (layer F.Cu) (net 6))
 (segment (start 55.35422 95.8342) (end 55.35422 83.26628) (width 0.25) (layer F.Cu) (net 6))
 (segment (start 53.5686 81.48066) (end 52.83454 81.48066) (width 0.25) (layer F.Cu) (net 6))
 (segment (start 55.35422 83.26628) (end 53.5686 81.48066) (width 0.25) (layer F.Cu) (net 6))
 (segment (start 86.693322 91.073281) (end 86.737461 91.11742) (width 0.25) (layer F.Cu) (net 7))
 (segment (start 85.10132 91.073281) (end 86.693322 91.073281) (width 0.25) (layer F.Cu) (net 7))
 (segment (start 86.737461 91.11742) (end 88.14562 91.11742) (width 0.25) (layer F.Cu) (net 7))
 (segment (start 88.14562 91.11742) (end 89.63152 92.60332) (width 0.25) (layer F.Cu) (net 7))
 (segment (start 89.63152 92.60332) (end 89.63152 116.31422) (width 0.25) (layer F.Cu) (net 7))
 (segment (start 89.63152 116.31422) (end 87.36584 118.5799) (width 0.25) (layer F.Cu) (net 7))
 (segment (start 87.36584 118.5799) (end 58.8264 118.5799) (width 0.25) (layer F.Cu) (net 7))
 (segment (start 58.8264 118.5799) (end 57.53862 117.29212) (width 0.25) (layer F.Cu) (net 7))
 (segment (start 54.42966 117.29212) (end 52.06746 119.65432) (width 0.25) (layer F.Cu) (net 7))
 (segment (start 57.53862 117.29212) (end 54.42966 117.29212) (width 0.25) (layer F.Cu) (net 7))
 (segment (start 52.06746 119.65432) (end 52.06746 113.15432) (width 0.25) (layer F.Cu) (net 7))
 (segment (start 85.10132 98.693281) (end 76.173019 98.693281) (width 0.25) (layer F.Cu) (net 8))
 (segment (start 76.173019 98.693281) (end 74.82078 100.04552) (width 0.25) (layer F.Cu) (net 8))
 (segment (start 74.82078 100.04552) (end 63.97498 100.04552) (width 0.25) (layer F.Cu) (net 8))
 (segment (start 61.37402 102.64648) (end 61.37402 104.3178) (width 0.25) (layer F.Cu) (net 8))
 (segment (start 63.97498 100.04552) (end 61.37402 102.64648) (width 0.25) (layer F.Cu) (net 8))
 (segment (start 59.78187 105.90995) (end 41.24495 105.90995) (width 0.25) (layer F.Cu) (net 8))
 (segment (start 61.37402 104.3178) (end 59.78187 105.90995) (width 0.25) (layer F.Cu) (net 8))
 (segment (start 38.52418 108.63072) (end 35.64128 108.63072) (width 0.25) (layer F.Cu) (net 8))
 (segment (start 41.24495 105.90995) (end 38.52418 108.63072) (width 0.25) (layer F.Cu) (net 8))
 (segment (start 76.89934 102.68628) (end 64.26792 102.68628) (width 0.25) (layer F.Cu) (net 9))
 (segment (start 85.10132 101.233281) (end 78.352339 101.233281) (width 0.25) (layer F.Cu) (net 9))
 (segment (start 78.352339 101.233281) (end 76.89934 102.68628) (width 0.25) (layer F.Cu) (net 9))
 (segment (start 64.26792 102.68628) (end 60.59424 106.35996) (width 0.25) (layer F.Cu) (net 9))
 (segment (start 60.59424 106.35996) (end 42.39514 106.35996) (width 0.25) (layer F.Cu) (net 9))
 (segment (start 37.58438 111.17072) (end 35.64128 111.17072) (width 0.25) (layer F.Cu) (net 9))
 (segment (start 42.39514 106.35996) (end 37.58438 111.17072) (width 0.25) (layer F.Cu) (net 9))
 (segment (start 63.244538 104.860282) (end 61.04171 107.06311) (width 0.25) (layer F.Cu) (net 10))
 (segment (start 85.10132 103.773281) (end 84.014319 104.860282) (width 0.25) (layer F.Cu) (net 10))
 (segment (start 84.014319 104.860282) (end 63.244538 104.860282) (width 0.25) (layer F.Cu) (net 10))
 (segment (start 42.534878 107.05571) (end 40.60952 108.981068) (width 0.25) (layer F.Cu) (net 10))
 (segment (start 52.416639 107.055709) (end 42.534878 107.05571) (width 0.25) (layer F.Cu) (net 10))
 (segment (start 61.04171 107.06311) (end 52.42404 107.06311) (width 0.25) (layer F.Cu) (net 10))
 (segment (start 52.42404 107.06311) (end 52.416639 107.055709) (width 0.25) (layer F.Cu) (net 10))
 (segment (start 40.60952 108.981068) (end 40.60952 110.00232) (width 0.25) (layer F.Cu) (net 10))
 (segment (start 36.90112 113.71072) (end 35.64128 113.71072) (width 0.25) (layer F.Cu) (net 10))
 (segment (start 40.60952 110.00232) (end 36.90112 113.71072) (width 0.25) (layer F.Cu) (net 10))
 (segment (start 35.64128 116.25072) (end 41.24198 110.65002) (width 0.25) (layer F.Cu) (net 11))
 (segment (start 42.721279 107.505719) (end 52.230239 107.505719) (width 0.25) (layer F.Cu) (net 11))
 (segment (start 41.24198 110.65002) (end 41.24198 108.985018) (width 0.25) (layer F.Cu) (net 11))
 (segment (start 41.24198 108.985018) (end 42.721279 107.505719) (width 0.25) (layer F.Cu) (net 11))
 (segment (start 52.230239 107.505719) (end 52.23764 107.51312) (width 0.25) (layer F.Cu) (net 11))
 (segment (start 52.23764 107.51312) (end 82.17662 107.51312) (width 0.25) (layer F.Cu) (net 11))
 (segment (start 83.376459 106.313281) (end 85.10132 106.313281) (width 0.25) (layer F.Cu) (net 11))
 (segment (start 82.17662 107.51312) (end 83.376459 106.313281) (width 0.25) (layer F.Cu) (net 11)))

